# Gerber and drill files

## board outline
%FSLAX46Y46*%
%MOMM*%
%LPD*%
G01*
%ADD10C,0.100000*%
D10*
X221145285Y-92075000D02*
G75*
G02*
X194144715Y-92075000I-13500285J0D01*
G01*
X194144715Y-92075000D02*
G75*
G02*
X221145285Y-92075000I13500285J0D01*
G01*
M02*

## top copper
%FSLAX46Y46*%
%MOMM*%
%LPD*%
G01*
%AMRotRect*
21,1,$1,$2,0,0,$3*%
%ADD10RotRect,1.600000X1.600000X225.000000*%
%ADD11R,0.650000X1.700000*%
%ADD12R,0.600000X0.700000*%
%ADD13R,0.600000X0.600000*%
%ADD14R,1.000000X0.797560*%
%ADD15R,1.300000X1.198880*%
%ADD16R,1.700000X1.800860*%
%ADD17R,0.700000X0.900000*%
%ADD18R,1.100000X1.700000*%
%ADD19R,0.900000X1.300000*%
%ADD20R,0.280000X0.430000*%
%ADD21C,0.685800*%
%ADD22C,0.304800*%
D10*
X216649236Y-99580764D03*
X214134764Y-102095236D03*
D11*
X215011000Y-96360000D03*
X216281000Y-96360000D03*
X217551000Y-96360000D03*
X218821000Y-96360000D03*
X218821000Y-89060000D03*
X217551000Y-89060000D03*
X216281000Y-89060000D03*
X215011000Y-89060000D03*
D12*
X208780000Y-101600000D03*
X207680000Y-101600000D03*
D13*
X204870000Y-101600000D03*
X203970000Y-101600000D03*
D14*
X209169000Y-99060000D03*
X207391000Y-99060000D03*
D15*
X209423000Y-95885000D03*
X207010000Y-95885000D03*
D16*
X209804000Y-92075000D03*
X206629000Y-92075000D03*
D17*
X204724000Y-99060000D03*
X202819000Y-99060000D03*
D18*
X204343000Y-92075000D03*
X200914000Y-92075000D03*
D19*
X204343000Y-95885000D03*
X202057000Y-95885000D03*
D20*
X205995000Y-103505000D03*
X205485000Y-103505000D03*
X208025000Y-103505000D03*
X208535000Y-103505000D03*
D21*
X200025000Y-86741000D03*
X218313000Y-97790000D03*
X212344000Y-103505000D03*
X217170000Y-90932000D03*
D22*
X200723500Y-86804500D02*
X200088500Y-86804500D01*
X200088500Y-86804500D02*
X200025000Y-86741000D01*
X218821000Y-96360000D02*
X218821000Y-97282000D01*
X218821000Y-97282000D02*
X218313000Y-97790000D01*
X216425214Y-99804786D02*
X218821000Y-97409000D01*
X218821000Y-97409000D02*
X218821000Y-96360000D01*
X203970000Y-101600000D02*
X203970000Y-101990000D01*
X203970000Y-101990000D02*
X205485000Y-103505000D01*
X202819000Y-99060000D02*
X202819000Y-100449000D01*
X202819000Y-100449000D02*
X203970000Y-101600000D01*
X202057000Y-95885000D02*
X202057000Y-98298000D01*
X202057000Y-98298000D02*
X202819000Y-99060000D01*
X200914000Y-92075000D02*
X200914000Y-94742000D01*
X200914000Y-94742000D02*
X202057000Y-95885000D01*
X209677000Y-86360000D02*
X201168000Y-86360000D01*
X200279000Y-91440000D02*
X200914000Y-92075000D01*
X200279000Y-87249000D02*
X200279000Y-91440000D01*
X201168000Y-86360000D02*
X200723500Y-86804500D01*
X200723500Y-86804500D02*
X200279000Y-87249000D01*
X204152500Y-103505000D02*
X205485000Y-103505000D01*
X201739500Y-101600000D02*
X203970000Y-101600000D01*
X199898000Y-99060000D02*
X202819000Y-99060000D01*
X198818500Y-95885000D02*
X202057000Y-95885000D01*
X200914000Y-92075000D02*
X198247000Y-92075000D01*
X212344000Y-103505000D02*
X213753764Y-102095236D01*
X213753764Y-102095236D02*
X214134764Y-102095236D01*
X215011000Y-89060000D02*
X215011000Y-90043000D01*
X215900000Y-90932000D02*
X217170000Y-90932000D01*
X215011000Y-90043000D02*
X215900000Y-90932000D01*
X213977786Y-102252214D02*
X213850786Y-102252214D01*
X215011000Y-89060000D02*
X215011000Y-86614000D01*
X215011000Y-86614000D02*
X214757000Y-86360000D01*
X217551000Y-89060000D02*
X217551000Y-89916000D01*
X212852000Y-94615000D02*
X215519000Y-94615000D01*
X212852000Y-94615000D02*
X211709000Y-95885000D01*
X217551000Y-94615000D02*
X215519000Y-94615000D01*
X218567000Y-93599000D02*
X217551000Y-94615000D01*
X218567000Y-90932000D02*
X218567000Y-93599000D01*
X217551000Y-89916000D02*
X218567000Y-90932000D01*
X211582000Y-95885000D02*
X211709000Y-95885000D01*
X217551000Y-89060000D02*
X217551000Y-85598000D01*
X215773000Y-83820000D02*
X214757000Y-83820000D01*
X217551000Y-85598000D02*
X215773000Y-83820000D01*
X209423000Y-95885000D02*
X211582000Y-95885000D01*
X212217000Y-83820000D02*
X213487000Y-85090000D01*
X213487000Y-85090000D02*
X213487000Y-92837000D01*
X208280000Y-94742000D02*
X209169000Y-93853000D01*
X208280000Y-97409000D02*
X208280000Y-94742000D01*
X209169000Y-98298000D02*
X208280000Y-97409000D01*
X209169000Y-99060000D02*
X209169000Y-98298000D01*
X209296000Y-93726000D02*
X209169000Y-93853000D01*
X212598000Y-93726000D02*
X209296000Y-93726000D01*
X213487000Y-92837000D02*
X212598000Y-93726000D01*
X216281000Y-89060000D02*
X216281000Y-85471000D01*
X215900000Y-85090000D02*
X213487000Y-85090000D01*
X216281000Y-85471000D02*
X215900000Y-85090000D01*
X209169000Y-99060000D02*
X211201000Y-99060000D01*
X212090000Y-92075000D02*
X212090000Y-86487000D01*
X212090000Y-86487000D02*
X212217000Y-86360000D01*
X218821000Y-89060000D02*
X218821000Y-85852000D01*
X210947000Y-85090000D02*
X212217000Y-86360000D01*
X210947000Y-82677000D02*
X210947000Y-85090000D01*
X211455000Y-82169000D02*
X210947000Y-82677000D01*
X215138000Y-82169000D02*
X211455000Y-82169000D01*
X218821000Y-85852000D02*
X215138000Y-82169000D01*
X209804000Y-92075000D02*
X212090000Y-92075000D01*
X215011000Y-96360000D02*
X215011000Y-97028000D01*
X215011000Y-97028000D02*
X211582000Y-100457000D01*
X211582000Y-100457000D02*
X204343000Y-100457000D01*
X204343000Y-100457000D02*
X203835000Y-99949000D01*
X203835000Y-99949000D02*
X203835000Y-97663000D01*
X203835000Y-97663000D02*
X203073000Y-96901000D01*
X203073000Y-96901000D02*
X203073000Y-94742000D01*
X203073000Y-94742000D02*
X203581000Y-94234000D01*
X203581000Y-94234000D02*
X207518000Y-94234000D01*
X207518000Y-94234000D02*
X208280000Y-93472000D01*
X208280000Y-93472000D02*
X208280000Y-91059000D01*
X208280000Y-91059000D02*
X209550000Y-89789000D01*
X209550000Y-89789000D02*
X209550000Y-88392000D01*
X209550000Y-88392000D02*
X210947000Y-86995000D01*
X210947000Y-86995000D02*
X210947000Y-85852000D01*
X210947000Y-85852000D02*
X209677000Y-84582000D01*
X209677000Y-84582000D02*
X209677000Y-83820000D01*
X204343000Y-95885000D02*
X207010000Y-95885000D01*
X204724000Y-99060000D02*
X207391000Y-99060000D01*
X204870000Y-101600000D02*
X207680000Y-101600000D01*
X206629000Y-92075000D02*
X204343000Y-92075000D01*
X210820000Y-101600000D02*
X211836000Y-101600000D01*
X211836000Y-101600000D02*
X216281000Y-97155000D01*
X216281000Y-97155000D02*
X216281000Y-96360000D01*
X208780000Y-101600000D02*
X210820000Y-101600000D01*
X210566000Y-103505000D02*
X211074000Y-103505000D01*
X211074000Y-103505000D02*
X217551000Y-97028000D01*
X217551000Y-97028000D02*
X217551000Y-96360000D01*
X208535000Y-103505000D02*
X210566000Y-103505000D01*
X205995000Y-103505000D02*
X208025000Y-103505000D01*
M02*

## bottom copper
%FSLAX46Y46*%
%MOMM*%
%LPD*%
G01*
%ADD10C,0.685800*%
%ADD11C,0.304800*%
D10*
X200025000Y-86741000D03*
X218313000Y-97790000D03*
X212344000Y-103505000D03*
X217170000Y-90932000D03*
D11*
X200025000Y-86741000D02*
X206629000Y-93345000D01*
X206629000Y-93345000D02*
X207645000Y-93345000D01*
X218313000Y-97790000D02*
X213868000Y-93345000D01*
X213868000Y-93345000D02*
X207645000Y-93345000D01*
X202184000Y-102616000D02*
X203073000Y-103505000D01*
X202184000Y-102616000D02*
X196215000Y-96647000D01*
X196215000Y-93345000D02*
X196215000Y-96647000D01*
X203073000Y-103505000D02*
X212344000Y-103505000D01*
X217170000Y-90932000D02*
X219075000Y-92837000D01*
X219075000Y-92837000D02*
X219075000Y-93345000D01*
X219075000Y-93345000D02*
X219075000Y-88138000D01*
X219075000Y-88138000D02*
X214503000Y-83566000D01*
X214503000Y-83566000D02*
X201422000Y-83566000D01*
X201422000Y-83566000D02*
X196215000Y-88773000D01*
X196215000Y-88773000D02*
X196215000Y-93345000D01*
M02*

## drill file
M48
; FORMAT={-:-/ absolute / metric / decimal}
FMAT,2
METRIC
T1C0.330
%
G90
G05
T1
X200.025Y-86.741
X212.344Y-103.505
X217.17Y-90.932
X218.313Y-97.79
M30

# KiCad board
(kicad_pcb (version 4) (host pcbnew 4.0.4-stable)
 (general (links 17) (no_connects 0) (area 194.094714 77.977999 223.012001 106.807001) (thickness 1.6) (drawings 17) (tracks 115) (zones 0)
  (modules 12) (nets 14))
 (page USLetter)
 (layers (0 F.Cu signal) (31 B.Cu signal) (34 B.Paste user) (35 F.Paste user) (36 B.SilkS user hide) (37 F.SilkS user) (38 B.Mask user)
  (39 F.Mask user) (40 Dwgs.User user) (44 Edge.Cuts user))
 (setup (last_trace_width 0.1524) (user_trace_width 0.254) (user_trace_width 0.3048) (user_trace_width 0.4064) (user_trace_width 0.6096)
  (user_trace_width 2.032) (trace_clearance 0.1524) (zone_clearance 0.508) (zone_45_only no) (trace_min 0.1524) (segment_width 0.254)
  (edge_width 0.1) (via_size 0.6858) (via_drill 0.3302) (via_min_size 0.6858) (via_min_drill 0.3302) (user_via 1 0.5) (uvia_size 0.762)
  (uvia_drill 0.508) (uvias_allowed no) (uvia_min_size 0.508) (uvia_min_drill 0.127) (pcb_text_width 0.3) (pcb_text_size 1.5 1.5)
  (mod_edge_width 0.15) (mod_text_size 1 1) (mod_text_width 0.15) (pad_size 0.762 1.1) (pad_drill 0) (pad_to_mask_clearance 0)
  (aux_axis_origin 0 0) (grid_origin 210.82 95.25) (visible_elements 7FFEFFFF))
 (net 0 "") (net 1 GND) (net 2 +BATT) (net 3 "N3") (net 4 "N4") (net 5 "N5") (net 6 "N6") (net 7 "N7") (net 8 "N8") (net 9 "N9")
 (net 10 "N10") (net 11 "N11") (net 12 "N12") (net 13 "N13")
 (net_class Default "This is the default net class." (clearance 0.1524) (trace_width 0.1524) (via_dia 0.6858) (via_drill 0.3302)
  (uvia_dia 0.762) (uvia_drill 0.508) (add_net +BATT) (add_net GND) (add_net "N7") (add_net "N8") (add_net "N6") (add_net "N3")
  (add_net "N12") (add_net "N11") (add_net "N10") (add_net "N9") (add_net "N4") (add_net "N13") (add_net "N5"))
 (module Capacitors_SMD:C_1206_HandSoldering (layer F.Cu) (at 215.392 100.838 225)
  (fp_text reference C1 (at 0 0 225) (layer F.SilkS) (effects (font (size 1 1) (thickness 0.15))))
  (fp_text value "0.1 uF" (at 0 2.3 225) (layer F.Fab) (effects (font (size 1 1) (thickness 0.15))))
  (pad 1 smd rect (at -1.778 0 225) (size 1.6 1.6) (layers F.Cu F.Paste F.Mask) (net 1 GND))
  (pad 2 smd rect (at 1.778 0 225) (size 1.6 1.6) (layers F.Cu F.Paste F.Mask) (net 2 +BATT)))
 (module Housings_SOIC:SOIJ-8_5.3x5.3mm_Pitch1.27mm (layer F.Cu) (at 216.916 92.71 90)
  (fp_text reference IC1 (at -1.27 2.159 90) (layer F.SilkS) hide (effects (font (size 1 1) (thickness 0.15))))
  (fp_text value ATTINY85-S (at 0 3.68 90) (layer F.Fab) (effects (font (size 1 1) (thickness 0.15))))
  (pad 1 smd rect (at -3.65 -1.905 90) (size 1.7 0.65) (layers F.Cu F.Paste F.Mask) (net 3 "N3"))
  (pad 2 smd rect (at -3.65 -0.635 90) (size 1.7 0.65) (layers F.Cu F.Paste F.Mask) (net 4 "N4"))
  (pad 3 smd rect (at -3.65 0.635 90) (size 1.7 0.65) (layers F.Cu F.Paste F.Mask) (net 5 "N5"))
  (pad 4 smd rect (at -3.65 1.905 90) (size 1.7 0.65) (layers F.Cu F.Paste F.Mask) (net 1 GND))
  (pad 5 smd rect (at 3.65 1.905 90) (size 1.7 0.65) (layers F.Cu F.Paste F.Mask) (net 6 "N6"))
  (pad 6 smd rect (at 3.65 0.635 90) (size 1.7 0.65) (layers F.Cu F.Paste F.Mask) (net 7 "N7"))
  (pad 7 smd rect (at 3.65 -0.635 90) (size 1.7 0.65) (layers F.Cu F.Paste F.Mask) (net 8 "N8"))
  (pad 8 smd rect (at 3.65 -1.905 90) (size 1.7 0.65) (layers F.Cu F.Paste F.Mask) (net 2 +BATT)))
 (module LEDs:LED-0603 (layer F.Cu) (at 208.28 101.6)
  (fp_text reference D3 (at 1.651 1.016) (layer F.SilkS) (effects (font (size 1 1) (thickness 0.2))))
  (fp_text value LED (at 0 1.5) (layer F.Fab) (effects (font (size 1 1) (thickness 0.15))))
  (pad 2 smd rect (at 0.5 0 180) (size 0.6 0.7) (layers F.Cu F.Paste F.Mask) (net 4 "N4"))
  (pad 1 smd rect (at -0.6 0 180) (size 0.6 0.7) (layers F.Cu F.Paste F.Mask) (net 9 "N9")))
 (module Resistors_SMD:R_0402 (layer F.Cu) (at 204.47 101.6 180)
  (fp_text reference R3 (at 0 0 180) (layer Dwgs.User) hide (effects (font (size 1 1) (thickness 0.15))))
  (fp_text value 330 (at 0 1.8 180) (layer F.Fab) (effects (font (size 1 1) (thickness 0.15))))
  (pad 1 smd rect (at -0.4 0 180) (size 0.6 0.6) (layers F.Cu F.Paste F.Mask) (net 9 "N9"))
  (pad 2 smd rect (at 0.5 0 180) (size 0.6 0.6) (layers F.Cu F.Paste F.Mask) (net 1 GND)))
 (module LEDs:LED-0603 (layer F.Cu) (at 208.28 99.06)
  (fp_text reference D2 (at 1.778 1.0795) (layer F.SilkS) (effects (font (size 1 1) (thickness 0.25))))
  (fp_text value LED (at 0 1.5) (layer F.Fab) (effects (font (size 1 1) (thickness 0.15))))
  (pad 2 smd rect (at 0.889 0 180) (size 1 0.79756) (layers F.Cu F.Paste F.Mask) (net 8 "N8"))
  (pad 1 smd rect (at -0.889 0 180) (size 1 0.79756) (layers F.Cu F.Paste F.Mask) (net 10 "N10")))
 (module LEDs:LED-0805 (layer F.Cu) (at 208.28 95.885)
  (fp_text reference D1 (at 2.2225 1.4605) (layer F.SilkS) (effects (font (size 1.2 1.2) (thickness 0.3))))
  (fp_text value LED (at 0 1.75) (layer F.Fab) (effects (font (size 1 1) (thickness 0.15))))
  (pad 2 smd rect (at 1.143 0 180) (size 1.3 1.19888) (layers F.Cu F.Paste F.Mask) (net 7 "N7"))
  (pad 1 smd rect (at -1.27 0 180) (size 1.3 1.19888) (layers F.Cu F.Paste F.Mask) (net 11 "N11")))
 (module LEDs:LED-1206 (layer F.Cu) (at 208.28 92.075)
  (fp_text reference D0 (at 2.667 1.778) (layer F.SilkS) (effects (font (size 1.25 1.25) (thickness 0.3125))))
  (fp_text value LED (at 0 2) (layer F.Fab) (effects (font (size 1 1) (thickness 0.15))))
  (pad 2 smd rect (at 1.524 0 180) (size 1.7 1.80086) (layers F.Cu F.Paste F.Mask) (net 6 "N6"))
  (pad 1 smd rect (at -1.651 0 180) (size 1.7 1.80086) (layers F.Cu F.Paste F.Mask) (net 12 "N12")))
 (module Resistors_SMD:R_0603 (layer F.Cu) (at 203.835 99.06 180)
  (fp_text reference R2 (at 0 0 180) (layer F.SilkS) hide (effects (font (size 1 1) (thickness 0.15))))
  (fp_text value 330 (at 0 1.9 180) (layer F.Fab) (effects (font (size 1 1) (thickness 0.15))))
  (pad 1 smd rect (at -0.889 0 180) (size 0.7 0.9) (layers F.Cu F.Paste F.Mask) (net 10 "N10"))
  (pad 2 smd rect (at 1.016 0 180) (size 0.7 0.9) (layers F.Cu F.Paste F.Mask) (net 1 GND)))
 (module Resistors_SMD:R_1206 (layer F.Cu) (at 202.565 92.075 180)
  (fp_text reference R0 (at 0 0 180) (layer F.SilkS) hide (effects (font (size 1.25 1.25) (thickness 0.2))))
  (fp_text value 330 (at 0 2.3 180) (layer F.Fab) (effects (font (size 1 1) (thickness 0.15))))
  (pad 1 smd rect (at -1.778 0 180) (size 1.1 1.7) (layers F.Cu F.Paste F.Mask) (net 12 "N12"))
  (pad 2 smd rect (at 1.651 0 180) (size 1.1 1.7) (layers F.Cu F.Paste F.Mask) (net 1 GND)))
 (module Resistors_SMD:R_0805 (layer F.Cu) (at 203.2 95.885 180)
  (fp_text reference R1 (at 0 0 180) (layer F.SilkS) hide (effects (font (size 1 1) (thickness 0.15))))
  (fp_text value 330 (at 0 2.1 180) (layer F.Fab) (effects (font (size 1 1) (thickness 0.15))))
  (pad 1 smd rect (at -1.143 0 180) (size 0.9 1.3) (layers F.Cu F.Paste F.Mask) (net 11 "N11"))
  (pad 2 smd rect (at 1.143 0 180) (size 0.9 1.3) (layers F.Cu F.Paste F.Mask) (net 1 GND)))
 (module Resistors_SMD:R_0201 (layer F.Cu) (at 205.74 103.505 180)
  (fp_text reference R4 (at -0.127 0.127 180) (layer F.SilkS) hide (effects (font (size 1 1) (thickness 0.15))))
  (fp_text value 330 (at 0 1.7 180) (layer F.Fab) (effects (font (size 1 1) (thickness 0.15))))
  (pad 1 smd rect (at -0.255 0 180) (size 0.28 0.43) (layers F.Cu F.Paste F.Mask) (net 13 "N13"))
  (pad 2 smd rect (at 0.255 0 180) (size 0.28 0.43) (layers F.Cu F.Paste F.Mask) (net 1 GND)))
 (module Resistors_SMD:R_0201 (layer F.Cu) (at 208.28 103.505)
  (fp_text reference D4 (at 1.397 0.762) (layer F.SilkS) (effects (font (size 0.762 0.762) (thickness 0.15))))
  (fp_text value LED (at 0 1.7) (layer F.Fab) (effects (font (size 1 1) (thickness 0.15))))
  (pad 1 smd rect (at -0.255 0) (size 0.28 0.43) (layers F.Cu F.Paste F.Mask) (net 13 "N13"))
  (pad 2 smd rect (at 0.255 0) (size 0.28 0.43) (layers F.Cu F.Paste F.Mask) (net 5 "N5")))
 (gr_circle (center 207.645 92.075) (end 197.485 83.185) (layer Edge.Cuts) (width 0.1))
 (segment (start 200.7235 86.8045) (end 200.0885 86.8045) (width 0.3048) (layer F.Cu) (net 1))
 (segment (start 200.025 86.741) (end 206.629 93.345) (width 0.3048) (layer B.Cu) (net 1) (status 20))
 (via (at 200.025 86.741) (size 0.6858) (drill 0.3302) (layers F.Cu B.Cu) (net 1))
 (segment (start 200.0885 86.8045) (end 200.025 86.741) (width 0.3048) (layer F.Cu) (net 1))
 (segment (start 206.629 93.345) (end 207.645 93.345) (width 0.3048) (layer B.Cu) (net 1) (status 30))
 (segment (start 218.821 96.36) (end 218.821 97.282) (width 0.3048) (layer F.Cu) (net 1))
 (segment (start 218.313 97.79) (end 213.868 93.345) (width 0.3048) (layer B.Cu) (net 1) (status 20))
 (via (at 218.313 97.79) (size 0.6858) (drill 0.3302) (layers F.Cu B.Cu) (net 1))
 (segment (start 218.821 97.282) (end 218.313 97.79) (width 0.3048) (layer F.Cu) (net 1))
 (segment (start 213.868 93.345) (end 207.645 93.345) (width 0.3048) (layer B.Cu) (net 1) (status 30))
 (segment (start 216.425214 99.804786) (end 218.821 97.409) (width 0.3048) (layer F.Cu) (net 1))
 (segment (start 218.821 97.409) (end 218.821 96.36) (width 0.3048) (layer F.Cu) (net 1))
 (segment (start 203.97 101.6) (end 203.97 101.99) (width 0.3048) (layer F.Cu) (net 1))
 (segment (start 203.97 101.99) (end 205.485 103.505) (width 0.3048) (layer F.Cu) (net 1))
 (segment (start 202.819 99.06) (end 202.819 100.449) (width 0.3048) (layer F.Cu) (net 1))
 (segment (start 202.819 100.449) (end 203.97 101.6) (width 0.3048) (layer F.Cu) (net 1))
 (segment (start 202.057 95.885) (end 202.057 98.298) (width 0.3048) (layer F.Cu) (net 1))
 (segment (start 202.057 98.298) (end 202.819 99.06) (width 0.3048) (layer F.Cu) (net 1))
 (segment (start 200.914 92.075) (end 200.914 94.742) (width 0.3048) (layer F.Cu) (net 1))
 (segment (start 200.914 94.742) (end 202.057 95.885) (width 0.3048) (layer F.Cu) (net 1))
 (segment (start 209.677 86.36) (end 201.168 86.36) (width 0.3048) (layer F.Cu) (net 1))
 (segment (start 200.279 91.44) (end 200.914 92.075) (width 0.3048) (layer F.Cu) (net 1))
 (segment (start 200.279 87.249) (end 200.279 91.44) (width 0.3048) (layer F.Cu) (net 1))
 (segment (start 201.168 86.36) (end 200.7235 86.8045) (width 0.3048) (layer F.Cu) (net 1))
 (segment (start 200.7235 86.8045) (end 200.279 87.249) (width 0.3048) (layer F.Cu) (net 1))
 (segment (start 204.1525 103.505) (end 205.485 103.505) (width 0.3048) (layer F.Cu) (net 1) (status 10))
 (segment (start 201.7395 101.6) (end 203.97 101.6) (width 0.3048) (layer F.Cu) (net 1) (status 10))
 (segment (start 199.898 99.06) (end 202.819 99.06) (width 0.3048) (layer F.Cu) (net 1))
 (segment (start 198.8185 95.885) (end 202.057 95.885) (width 0.3048) (layer F.Cu) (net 1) (status 10))
 (segment (start 200.914 92.075) (end 198.247 92.075) (width 0.3048) (layer F.Cu) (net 1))
 (segment (start 202.184 102.616) (end 203.073 103.505) (width 0.3048) (layer B.Cu) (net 2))
 (segment (start 202.184 102.616) (end 196.215 96.647) (width 0.3048) (layer B.Cu) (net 2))
 (segment (start 196.215 93.345) (end 196.215 96.647) (width 0.3048) (layer B.Cu) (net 2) (status 10))
 (segment (start 212.344 103.505) (end 213.753764 102.095236) (width 0.3048) (layer F.Cu) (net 2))
 (via (at 212.344 103.505) (size 0.6858) (drill 0.3302) (layers F.Cu B.Cu) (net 2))
 (segment (start 203.073 103.505) (end 212.344 103.505) (width 0.3048) (layer B.Cu) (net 2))
 (segment (start 213.753764 102.095236) (end 214.134764 102.095236) (width 0.3048) (layer F.Cu) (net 2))
 (segment (start 215.011 89.06) (end 215.011 90.043) (width 0.3048) (layer F.Cu) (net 2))
 (segment (start 217.17 90.932) (end 219.075 92.837) (width 0.3048) (layer B.Cu) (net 2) (status 20))
 (via (at 217.17 90.932) (size 0.6858) (drill 0.3302) (layers F.Cu B.Cu) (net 2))
 (segment (start 215.9 90.932) (end 217.17 90.932) (width 0.3048) (layer F.Cu) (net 2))
 (segment (start 215.011 90.043) (end 215.9 90.932) (width 0.3048) (layer F.Cu) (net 2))
 (segment (start 219.075 92.837) (end 219.075 93.345) (width 0.3048) (layer B.Cu) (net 2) (status 30))
 (segment (start 219.075 93.345) (end 219.075 88.138) (width 0.3048) (layer B.Cu) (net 2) (status 10))
 (segment (start 219.075 88.138) (end 214.503 83.566) (width 0.3048) (layer B.Cu) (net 2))
 (segment (start 214.503 83.566) (end 201.422 83.566) (width 0.3048) (layer B.Cu) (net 2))
 (segment (start 201.422 83.566) (end 196.215 88.773) (width 0.3048) (layer B.Cu) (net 2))
 (segment (start 196.215 88.773) (end 196.215 93.345) (width 0.3048) (layer B.Cu) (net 2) (status 20))
 (segment (start 213.977786 102.252214) (end 213.850786 102.252214) (width 0.3048) (layer F.Cu) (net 2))
 (segment (start 215.011 89.06) (end 215.011 86.614) (width 0.3048) (layer F.Cu) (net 2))
 (segment (start 215.011 86.614) (end 214.757 86.36) (width 0.3048) (layer F.Cu) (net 2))
 (segment (start 217.551 89.06) (end 217.551 89.916) (width 0.3048) (layer F.Cu) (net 7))
 (segment (start 212.852 94.615) (end 215.519 94.615) (width 0.3048) (layer F.Cu) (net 7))
 (segment (start 212.852 94.615) (end 211.709 95.885) (width 0.3048) (layer F.Cu) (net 7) (status 20))
 (segment (start 217.551 94.615) (end 215.519 94.615) (width 0.3048) (layer F.Cu) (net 7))
 (segment (start 218.567 93.599) (end 217.551 94.615) (width 0.3048) (layer F.Cu) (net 7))
 (segment (start 218.567 90.932) (end 218.567 93.599) (width 0.3048) (layer F.Cu) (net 7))
 (segment (start 217.551 89.916) (end 218.567 90.932) (width 0.3048) (layer F.Cu) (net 7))
 (segment (start 211.582 95.885) (end 211.709 95.885) (width 0.3048) (layer F.Cu) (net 7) (status 30))
 (segment (start 217.551 89.06) (end 217.551 85.598) (width 0.3048) (layer F.Cu) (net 7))
 (segment (start 215.773 83.82) (end 214.757 83.82) (width 0.3048) (layer F.Cu) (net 7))
 (segment (start 217.551 85.598) (end 215.773 83.82) (width 0.3048) (layer F.Cu) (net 7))
 (segment (start 209.423 95.885) (end 211.582 95.885) (width 0.3048) (layer F.Cu) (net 7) (status 20))
 (segment (start 212.217 83.82) (end 213.487 85.09) (width 0.3048) (layer F.Cu) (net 8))
 (segment (start 213.487 85.09) (end 213.487 92.837) (width 0.3048) (layer F.Cu) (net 8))
 (segment (start 208.28 94.742) (end 209.169 93.853) (width 0.3048) (layer F.Cu) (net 8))
 (segment (start 208.28 97.409) (end 208.28 94.742) (width 0.3048) (layer F.Cu) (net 8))
 (segment (start 209.169 98.298) (end 208.28 97.409) (width 0.3048) (layer F.Cu) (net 8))
 (segment (start 209.169 99.06) (end 209.169 98.298) (width 0.3048) (layer F.Cu) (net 8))
 (segment (start 209.296 93.726) (end 209.169 93.853) (width 0.3048) (layer F.Cu) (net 8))
 (segment (start 212.598 93.726) (end 209.296 93.726) (width 0.3048) (layer F.Cu) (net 8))
 (segment (start 213.487 92.837) (end 212.598 93.726) (width 0.3048) (layer F.Cu) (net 8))
 (segment (start 216.281 89.06) (end 216.281 85.471) (width 0.3048) (layer F.Cu) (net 8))
 (segment (start 215.9 85.09) (end 213.487 85.09) (width 0.3048) (layer F.Cu) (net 8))
 (segment (start 216.281 85.471) (end 215.9 85.09) (width 0.3048) (layer F.Cu) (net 8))
 (segment (start 209.169 99.06) (end 211.201 99.06) (width 0.3048) (layer F.Cu) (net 8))
 (segment (start 212.09 92.075) (end 212.09 86.487) (width 0.3048) (layer F.Cu) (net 6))
 (segment (start 212.09 86.487) (end 212.217 86.36) (width 0.3048) (layer F.Cu) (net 6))
 (segment (start 218.821 89.06) (end 218.821 85.852) (width 0.3048) (layer F.Cu) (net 6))
 (segment (start 210.947 85.09) (end 212.217 86.36) (width 0.3048) (layer F.Cu) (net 6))
 (segment (start 210.947 82.677) (end 210.947 85.09) (width 0.3048) (layer F.Cu) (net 6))
 (segment (start 211.455 82.169) (end 210.947 82.677) (width 0.3048) (layer F.Cu) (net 6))
 (segment (start 215.138 82.169) (end 211.455 82.169) (width 0.3048) (layer F.Cu) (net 6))
 (segment (start 218.821 85.852) (end 215.138 82.169) (width 0.3048) (layer F.Cu) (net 6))
 (segment (start 209.804 92.075) (end 212.09 92.075) (width 0.3048) (layer F.Cu) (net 6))
 (segment (start 215.011 96.36) (end 215.011 97.028) (width 0.3048) (layer F.Cu) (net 3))
 (segment (start 215.011 97.028) (end 211.582 100.457) (width 0.3048) (layer F.Cu) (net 3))
 (segment (start 211.582 100.457) (end 204.343 100.457) (width 0.3048) (layer F.Cu) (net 3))
 (segment (start 204.343 100.457) (end 203.835 99.949) (width 0.3048) (layer F.Cu) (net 3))
 (segment (start 203.835 99.949) (end 203.835 97.663) (width 0.3048) (layer F.Cu) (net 3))
 (segment (start 203.835 97.663) (end 203.073 96.901) (width 0.3048) (layer F.Cu) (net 3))
 (segment (start 203.073 96.901) (end 203.073 94.742) (width 0.3048) (layer F.Cu) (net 3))
 (segment (start 203.073 94.742) (end 203.581 94.234) (width 0.3048) (layer F.Cu) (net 3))
 (segment (start 203.581 94.234) (end 207.518 94.234) (width 0.3048) (layer F.Cu) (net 3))
 (segment (start 207.518 94.234) (end 208.28 93.472) (width 0.3048) (layer F.Cu) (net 3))
 (segment (start 208.28 93.472) (end 208.28 91.059) (width 0.3048) (layer F.Cu) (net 3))
 (segment (start 208.28 91.059) (end 209.55 89.789) (width 0.3048) (layer F.Cu) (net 3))
 (segment (start 209.55 89.789) (end 209.55 88.392) (width 0.3048) (layer F.Cu) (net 3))
 (segment (start 209.55 88.392) (end 210.947 86.995) (width 0.3048) (layer F.Cu) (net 3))
 (segment (start 210.947 86.995) (end 210.947 85.852) (width 0.3048) (layer F.Cu) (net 3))
 (segment (start 210.947 85.852) (end 209.677 84.582) (width 0.3048) (layer F.Cu) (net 3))
 (segment (start 209.677 84.582) (end 209.677 83.82) (width 0.3048) (layer F.Cu) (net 3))
 (segment (start 204.343 95.885) (end 207.01 95.885) (width 0.3048) (layer F.Cu) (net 11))
 (segment (start 204.724 99.06) (end 207.391 99.06) (width 0.3048) (layer F.Cu) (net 10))
 (segment (start 204.87 101.6) (end 207.68 101.6) (width 0.3048) (layer F.Cu) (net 9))
 (segment (start 206.629 92.075) (end 204.343 92.075) (width 0.3048) (layer F.Cu) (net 12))
 (segment (start 210.82 101.6) (end 211.836 101.6) (width 0.3048) (layer F.Cu) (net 4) (status 10))
 (segment (start 211.836 101.6) (end 216.281 97.155) (width 0.3048) (layer F.Cu) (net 4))
 (segment (start 216.281 97.155) (end 216.281 96.36) (width 0.3048) (layer F.Cu) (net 4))
 (segment (start 208.78 101.6) (end 210.82 101.6) (width 0.3048) (layer F.Cu) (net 4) (status 20))
 (segment (start 210.566 103.505) (end 211.074 103.505) (width 0.3048) (layer F.Cu) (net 5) (status 10))
 (segment (start 211.074 103.505) (end 217.551 97.028) (width 0.3048) (layer F.Cu) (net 5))
 (segment (start 217.551 97.028) (end 217.551 96.36) (width 0.3048) (layer F.Cu) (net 5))
 (segment (start 208.535 103.505) (end 210.566 103.505) (width 0.3048) (layer F.Cu) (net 5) (status 20))
 (segment (start 205.995 103.505) (end 208.025 103.505) (width 0.3048) (layer F.Cu) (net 13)))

